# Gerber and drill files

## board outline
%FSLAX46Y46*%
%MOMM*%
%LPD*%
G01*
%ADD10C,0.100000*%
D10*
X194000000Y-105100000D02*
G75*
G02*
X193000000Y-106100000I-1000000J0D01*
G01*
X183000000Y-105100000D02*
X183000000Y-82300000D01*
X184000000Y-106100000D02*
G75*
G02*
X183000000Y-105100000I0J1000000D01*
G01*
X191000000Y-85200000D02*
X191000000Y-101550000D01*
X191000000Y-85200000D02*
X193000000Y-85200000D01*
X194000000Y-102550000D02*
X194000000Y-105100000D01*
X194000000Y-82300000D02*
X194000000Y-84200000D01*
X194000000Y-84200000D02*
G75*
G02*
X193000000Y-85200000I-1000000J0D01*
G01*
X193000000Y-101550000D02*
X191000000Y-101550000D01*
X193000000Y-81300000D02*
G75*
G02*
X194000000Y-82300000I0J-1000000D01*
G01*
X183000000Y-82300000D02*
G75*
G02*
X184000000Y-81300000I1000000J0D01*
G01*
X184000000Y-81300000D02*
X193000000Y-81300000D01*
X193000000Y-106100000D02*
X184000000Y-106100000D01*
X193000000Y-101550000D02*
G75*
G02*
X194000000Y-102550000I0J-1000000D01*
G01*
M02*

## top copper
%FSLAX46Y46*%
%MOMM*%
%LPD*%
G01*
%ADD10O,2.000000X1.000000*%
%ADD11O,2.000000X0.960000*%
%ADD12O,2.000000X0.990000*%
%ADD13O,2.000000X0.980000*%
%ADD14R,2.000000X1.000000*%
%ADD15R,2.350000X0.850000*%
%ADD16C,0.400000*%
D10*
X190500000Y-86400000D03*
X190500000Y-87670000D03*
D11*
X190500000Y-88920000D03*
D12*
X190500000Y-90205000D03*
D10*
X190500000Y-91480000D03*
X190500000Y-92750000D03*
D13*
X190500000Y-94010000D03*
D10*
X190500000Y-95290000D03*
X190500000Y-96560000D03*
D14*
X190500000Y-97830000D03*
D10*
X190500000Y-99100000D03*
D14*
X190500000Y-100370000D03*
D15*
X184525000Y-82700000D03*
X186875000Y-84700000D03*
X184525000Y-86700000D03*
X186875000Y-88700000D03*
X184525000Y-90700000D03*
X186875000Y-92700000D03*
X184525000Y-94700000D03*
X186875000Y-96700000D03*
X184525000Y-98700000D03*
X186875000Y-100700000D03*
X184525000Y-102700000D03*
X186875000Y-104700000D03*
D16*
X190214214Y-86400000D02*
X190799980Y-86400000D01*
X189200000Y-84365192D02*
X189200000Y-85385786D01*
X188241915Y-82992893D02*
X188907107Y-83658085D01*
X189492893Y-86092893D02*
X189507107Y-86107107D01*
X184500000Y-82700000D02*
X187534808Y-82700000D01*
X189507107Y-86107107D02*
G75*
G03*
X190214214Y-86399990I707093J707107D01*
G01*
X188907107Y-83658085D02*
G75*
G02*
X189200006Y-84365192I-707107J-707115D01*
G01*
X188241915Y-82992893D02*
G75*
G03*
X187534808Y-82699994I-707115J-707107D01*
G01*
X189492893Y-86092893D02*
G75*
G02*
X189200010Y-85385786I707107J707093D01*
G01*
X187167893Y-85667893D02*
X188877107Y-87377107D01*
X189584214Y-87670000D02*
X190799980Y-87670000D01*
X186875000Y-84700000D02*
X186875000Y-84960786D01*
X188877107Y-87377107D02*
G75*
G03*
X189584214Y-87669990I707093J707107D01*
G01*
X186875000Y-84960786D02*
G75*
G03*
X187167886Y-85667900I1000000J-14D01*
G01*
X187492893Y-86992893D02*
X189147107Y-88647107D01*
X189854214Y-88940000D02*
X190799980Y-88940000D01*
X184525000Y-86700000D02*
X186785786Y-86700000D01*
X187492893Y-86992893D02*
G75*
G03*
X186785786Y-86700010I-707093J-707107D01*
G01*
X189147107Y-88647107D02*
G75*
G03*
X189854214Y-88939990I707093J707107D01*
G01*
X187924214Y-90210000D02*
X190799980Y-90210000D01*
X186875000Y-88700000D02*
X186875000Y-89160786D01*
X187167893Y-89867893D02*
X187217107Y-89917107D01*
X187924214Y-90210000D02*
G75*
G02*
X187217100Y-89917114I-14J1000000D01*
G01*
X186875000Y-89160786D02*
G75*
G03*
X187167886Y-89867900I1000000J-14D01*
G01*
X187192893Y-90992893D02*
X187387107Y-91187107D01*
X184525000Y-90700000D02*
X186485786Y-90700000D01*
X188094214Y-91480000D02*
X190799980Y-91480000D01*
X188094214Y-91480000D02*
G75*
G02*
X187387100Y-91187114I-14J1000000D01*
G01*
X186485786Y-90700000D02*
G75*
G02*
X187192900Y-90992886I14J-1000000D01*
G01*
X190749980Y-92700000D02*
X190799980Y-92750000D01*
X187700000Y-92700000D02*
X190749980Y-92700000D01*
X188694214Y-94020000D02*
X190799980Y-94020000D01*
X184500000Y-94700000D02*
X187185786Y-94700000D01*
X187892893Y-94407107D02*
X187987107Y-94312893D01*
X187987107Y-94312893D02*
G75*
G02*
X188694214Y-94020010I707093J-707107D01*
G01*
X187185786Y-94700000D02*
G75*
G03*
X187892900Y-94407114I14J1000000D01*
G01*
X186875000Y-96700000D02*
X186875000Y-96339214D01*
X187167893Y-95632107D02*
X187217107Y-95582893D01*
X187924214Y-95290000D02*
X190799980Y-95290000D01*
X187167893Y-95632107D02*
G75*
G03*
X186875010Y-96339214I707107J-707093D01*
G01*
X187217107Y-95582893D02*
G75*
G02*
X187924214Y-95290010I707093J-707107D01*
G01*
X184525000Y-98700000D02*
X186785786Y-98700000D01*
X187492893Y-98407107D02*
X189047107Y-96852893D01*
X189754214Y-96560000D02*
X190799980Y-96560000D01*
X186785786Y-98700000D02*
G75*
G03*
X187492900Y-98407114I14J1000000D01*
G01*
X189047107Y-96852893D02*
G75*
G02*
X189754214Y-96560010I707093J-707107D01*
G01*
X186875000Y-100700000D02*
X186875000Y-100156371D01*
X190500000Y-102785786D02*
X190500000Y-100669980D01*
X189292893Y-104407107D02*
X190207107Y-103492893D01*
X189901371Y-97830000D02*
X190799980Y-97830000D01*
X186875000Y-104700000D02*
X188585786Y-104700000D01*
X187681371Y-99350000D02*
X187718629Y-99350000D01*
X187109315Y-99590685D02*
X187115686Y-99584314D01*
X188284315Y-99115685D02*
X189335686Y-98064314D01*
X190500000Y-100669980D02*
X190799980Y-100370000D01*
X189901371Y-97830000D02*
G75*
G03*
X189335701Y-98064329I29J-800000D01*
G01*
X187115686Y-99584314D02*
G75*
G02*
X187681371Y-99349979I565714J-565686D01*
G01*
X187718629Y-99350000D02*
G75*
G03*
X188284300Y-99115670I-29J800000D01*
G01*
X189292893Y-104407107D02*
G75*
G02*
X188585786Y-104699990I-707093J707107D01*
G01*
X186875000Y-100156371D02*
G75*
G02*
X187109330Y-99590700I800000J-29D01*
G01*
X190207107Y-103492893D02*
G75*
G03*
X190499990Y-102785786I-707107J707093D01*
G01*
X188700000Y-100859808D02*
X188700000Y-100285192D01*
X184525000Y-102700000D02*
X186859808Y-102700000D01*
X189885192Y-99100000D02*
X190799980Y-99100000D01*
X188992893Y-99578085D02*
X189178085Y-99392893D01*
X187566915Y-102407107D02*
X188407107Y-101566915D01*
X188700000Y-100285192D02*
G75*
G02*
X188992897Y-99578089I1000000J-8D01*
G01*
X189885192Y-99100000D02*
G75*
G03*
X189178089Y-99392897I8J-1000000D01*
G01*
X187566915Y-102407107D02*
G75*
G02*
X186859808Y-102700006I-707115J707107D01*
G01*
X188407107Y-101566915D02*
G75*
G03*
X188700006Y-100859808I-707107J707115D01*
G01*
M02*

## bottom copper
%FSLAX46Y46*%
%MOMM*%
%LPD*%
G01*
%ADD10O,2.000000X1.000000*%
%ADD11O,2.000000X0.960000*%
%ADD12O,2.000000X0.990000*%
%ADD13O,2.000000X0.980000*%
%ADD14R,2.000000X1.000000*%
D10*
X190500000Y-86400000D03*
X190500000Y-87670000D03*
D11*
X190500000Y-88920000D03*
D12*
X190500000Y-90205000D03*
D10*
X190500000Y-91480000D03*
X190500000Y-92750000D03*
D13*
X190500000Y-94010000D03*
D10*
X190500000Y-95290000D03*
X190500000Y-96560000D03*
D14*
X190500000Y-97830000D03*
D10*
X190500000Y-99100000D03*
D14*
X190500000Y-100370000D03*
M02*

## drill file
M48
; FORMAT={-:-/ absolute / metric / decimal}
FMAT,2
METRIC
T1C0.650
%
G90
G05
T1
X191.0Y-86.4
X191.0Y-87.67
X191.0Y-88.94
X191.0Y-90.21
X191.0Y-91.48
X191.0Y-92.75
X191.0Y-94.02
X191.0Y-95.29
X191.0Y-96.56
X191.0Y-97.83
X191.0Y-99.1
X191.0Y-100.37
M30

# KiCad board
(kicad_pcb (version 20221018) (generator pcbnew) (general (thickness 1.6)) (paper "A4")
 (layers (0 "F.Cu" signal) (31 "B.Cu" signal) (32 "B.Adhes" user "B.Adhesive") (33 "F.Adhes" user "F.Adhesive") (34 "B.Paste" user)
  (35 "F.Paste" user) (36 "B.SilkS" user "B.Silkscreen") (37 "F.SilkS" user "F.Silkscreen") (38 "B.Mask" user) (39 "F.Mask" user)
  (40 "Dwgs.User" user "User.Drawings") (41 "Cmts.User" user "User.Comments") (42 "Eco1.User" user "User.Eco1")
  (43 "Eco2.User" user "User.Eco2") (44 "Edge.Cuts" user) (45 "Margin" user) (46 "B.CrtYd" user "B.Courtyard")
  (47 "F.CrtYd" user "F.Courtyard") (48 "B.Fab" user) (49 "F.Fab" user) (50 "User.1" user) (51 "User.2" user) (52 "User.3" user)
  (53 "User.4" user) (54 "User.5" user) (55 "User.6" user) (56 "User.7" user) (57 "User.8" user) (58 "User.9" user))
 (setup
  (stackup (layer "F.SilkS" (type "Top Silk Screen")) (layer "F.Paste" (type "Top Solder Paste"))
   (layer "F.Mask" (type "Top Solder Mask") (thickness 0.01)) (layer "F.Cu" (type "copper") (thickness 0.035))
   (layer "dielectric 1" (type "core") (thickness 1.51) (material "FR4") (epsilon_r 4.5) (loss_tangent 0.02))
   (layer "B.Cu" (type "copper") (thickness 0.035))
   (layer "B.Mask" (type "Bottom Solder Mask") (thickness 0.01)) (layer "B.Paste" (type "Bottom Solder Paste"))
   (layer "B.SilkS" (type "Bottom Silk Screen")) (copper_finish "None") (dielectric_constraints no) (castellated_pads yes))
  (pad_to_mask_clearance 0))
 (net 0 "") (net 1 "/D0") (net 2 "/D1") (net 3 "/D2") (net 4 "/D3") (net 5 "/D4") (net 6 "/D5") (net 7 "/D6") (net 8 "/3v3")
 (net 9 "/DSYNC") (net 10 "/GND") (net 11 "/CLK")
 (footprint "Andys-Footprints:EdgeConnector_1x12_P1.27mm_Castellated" (layer "F.Cu") (at 191 86.4)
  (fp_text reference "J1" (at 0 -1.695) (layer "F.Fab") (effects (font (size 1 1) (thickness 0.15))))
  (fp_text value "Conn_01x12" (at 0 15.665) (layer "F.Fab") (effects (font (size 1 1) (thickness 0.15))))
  (pad "1" thru_hole oval (at 0 0) (size 2 1) (drill 0.65 (offset -0.5 0)) (layers "*.Cu" "*.Mask") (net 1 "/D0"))
  (pad "2" thru_hole oval (at 0 1.27) (size 2 1) (drill 0.65 (offset -0.5 0)) (layers "*.Cu" "*.Mask") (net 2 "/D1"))
  (pad "3" thru_hole oval (at 0 2.54) (size 2 0.96) (drill 0.65 (offset -0.5 -0.02)) (layers "*.Cu" "*.Mask") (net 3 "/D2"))
  (pad "4" thru_hole oval (at 0 3.81) (size 2 0.99) (drill 0.65 (offset -0.5 -0.005)) (layers "*.Cu" "*.Mask") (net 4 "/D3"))
  (pad "5" thru_hole oval (at 0 5.08) (size 2 1) (drill 0.65 (offset -0.5 0)) (layers "*.Cu" "*.Mask") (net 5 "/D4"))
  (pad "6" thru_hole oval (at 0 6.35) (size 2 1) (drill 0.65 (offset -0.5 0)) (layers "*.Cu" "*.Mask") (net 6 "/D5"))
  (pad "7" thru_hole oval (at 0 7.62) (size 2 0.98) (drill 0.65 (offset -0.5 -0.01)) (layers "*.Cu" "*.Mask") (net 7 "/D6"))
  (pad "8" thru_hole oval (at 0 8.89) (size 2 1) (drill 0.65 (offset -0.5 0)) (layers "*.Cu" "*.Mask") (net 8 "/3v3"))
  (pad "9" thru_hole oval (at 0 10.16) (size 2 1) (drill 0.65 (offset -0.5 0)) (layers "*.Cu" "*.Mask") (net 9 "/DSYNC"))
  (pad "10" thru_hole rect (at 0 11.43) (size 2 1) (drill 0.65 (offset -0.5 0)) (layers "*.Cu" "*.Mask") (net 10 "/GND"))
  (pad "11" thru_hole oval (at 0 12.7) (size 2 1) (drill 0.65 (offset -0.5 0)) (layers "*.Cu" "*.Mask") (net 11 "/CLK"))
  (pad "12" thru_hole rect (at 0 13.97) (size 2 1) (drill 0.65 (offset -0.5 0)) (layers "*.Cu" "*.Mask") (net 10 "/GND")))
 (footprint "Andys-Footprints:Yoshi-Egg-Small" (layer "F.Cu") (at 191.7 103.8)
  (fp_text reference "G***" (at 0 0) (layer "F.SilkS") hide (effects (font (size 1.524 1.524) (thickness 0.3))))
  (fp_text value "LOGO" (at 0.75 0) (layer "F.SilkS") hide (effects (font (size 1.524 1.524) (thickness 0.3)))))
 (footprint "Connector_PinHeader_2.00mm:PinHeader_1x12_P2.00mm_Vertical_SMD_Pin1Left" (layer "F.Cu") (at 185.7 93.7)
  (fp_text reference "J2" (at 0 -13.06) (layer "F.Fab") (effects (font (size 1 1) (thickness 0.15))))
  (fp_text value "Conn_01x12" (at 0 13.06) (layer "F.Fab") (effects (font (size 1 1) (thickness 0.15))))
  (pad "1" smd rect (at -1.175 -11) (size 2.35 0.85) (layers "F.Cu" "F.Paste" "F.Mask") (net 1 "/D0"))
  (pad "2" smd rect (at 1.175 -9) (size 2.35 0.85) (layers "F.Cu" "F.Paste" "F.Mask") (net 2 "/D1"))
  (pad "3" smd rect (at -1.175 -7) (size 2.35 0.85) (layers "F.Cu" "F.Paste" "F.Mask") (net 3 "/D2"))
  (pad "4" smd rect (at 1.175 -5) (size 2.35 0.85) (layers "F.Cu" "F.Paste" "F.Mask") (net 4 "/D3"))
  (pad "5" smd rect (at -1.175 -3) (size 2.35 0.85) (layers "F.Cu" "F.Paste" "F.Mask") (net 5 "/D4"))
  (pad "6" smd rect (at 1.175 -1) (size 2.35 0.85) (layers "F.Cu" "F.Paste" "F.Mask") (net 6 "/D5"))
  (pad "7" smd rect (at -1.175 1) (size 2.35 0.85) (layers "F.Cu" "F.Paste" "F.Mask") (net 7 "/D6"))
  (pad "8" smd rect (at 1.175 3) (size 2.35 0.85) (layers "F.Cu" "F.Paste" "F.Mask") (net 8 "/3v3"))
  (pad "9" smd rect (at -1.175 5) (size 2.35 0.85) (layers "F.Cu" "F.Paste" "F.Mask") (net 9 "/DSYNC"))
  (pad "10" smd rect (at 1.175 7) (size 2.35 0.85) (layers "F.Cu" "F.Paste" "F.Mask") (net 10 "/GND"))
  (pad "11" smd rect (at -1.175 9) (size 2.35 0.85) (layers "F.Cu" "F.Paste" "F.Mask") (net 11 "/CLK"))
  (pad "12" smd rect (at 1.175 11) (size 2.35 0.85) (layers "F.Cu" "F.Paste" "F.Mask") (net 10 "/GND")))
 (gr_arc (start 194 105.1) (mid 193.707107 105.807107) (end 193 106.1) (stroke (width 0.1) (type solid)) (layer "Edge.Cuts"))
 (gr_line (start 183 105.1) (end 183 82.3) (stroke (width 0.1) (type solid)) (layer "Edge.Cuts"))
 (gr_arc (start 184 106.1) (mid 183.292893 105.807107) (end 183 105.1) (stroke (width 0.1) (type solid)) (layer "Edge.Cuts"))
 (gr_line (start 191 85.2) (end 191 101.55) (stroke (width 0.1) (type solid)) (layer "Edge.Cuts"))
 (gr_line (start 191 85.2) (end 193 85.2) (stroke (width 0.1) (type solid)) (layer "Edge.Cuts"))
 (gr_line (start 194 102.55) (end 194 105.1) (stroke (width 0.1) (type solid)) (layer "Edge.Cuts"))
 (gr_line (start 194 82.3) (end 194 84.2) (stroke (width 0.1) (type solid)) (layer "Edge.Cuts"))
 (gr_arc (start 194 84.2) (mid 193.707107 84.907107) (end 193 85.2) (stroke (width 0.1) (type solid)) (layer "Edge.Cuts"))
 (gr_line (start 193 101.55) (end 191 101.55) (stroke (width 0.1) (type solid)) (layer "Edge.Cuts"))
 (gr_arc (start 193 81.3) (mid 193.707107 81.592893) (end 194 82.3) (stroke (width 0.1) (type solid)) (layer "Edge.Cuts"))
 (gr_arc (start 183 82.3) (mid 183.292893 81.592893) (end 184 81.3) (stroke (width 0.1) (type solid)) (layer "Edge.Cuts"))
 (gr_line (start 184 81.3) (end 193 81.3) (stroke (width 0.1) (type solid)) (layer "Edge.Cuts"))
 (gr_line (start 193 106.1) (end 184 106.1) (stroke (width 0.1) (type solid)) (layer "Edge.Cuts"))
 (gr_arc (start 193 101.55) (mid 193.707107 101.842893) (end 194 102.55) (stroke (width 0.1) (type solid)) (layer "Edge.Cuts"))
 (segment (start 190.214214 86.4) (end 190.79998 86.4) (width 0.4) (layer "F.Cu") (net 1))
 (segment (start 189.2 84.365192) (end 189.2 85.385786) (width 0.4) (layer "F.Cu") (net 1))
 (segment (start 188.241915 82.992893) (end 188.907107 83.658085) (width 0.4) (layer "F.Cu") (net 1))
 (segment (start 189.492893 86.092893) (end 189.507107 86.107107) (width 0.4) (layer "F.Cu") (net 1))
 (segment (start 184.5 82.7) (end 187.534808 82.7) (width 0.4) (layer "F.Cu") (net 1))
 (arc (start 189.507107 86.107107) (mid 189.83153 86.32388) (end 190.214214 86.4) (width 0.4) (layer "F.Cu") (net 1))
 (arc (start 188.907107 83.658085) (mid 189.12388 83.982508) (end 189.2 84.365192) (width 0.4) (layer "F.Cu") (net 1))
 (arc (start 188.241915 82.992893) (mid 187.917492 82.77612) (end 187.534808 82.7) (width 0.4) (layer "F.Cu") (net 1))
 (arc (start 189.492893 86.092893) (mid 189.27612 85.76847) (end 189.2 85.385786) (width 0.4) (layer "F.Cu") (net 1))
 (segment (start 187.167893 85.667893) (end 188.877107 87.377107) (width 0.4) (layer "F.Cu") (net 2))
 (segment (start 189.584214 87.67) (end 190.79998 87.67) (width 0.4) (layer "F.Cu") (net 2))
 (segment (start 186.875 84.7) (end 186.875 84.960786) (width 0.4) (layer "F.Cu") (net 2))
 (arc (start 188.877107 87.377107) (mid 189.20153 87.59388) (end 189.584214 87.67) (width 0.4) (layer "F.Cu") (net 2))
 (arc (start 186.875 84.960786) (mid 186.95112 85.343469) (end 187.167893 85.667893) (width 0.4) (layer "F.Cu") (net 2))
 (segment (start 187.492893 86.992893) (end 189.147107 88.647107) (width 0.4) (layer "F.Cu") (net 3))
 (segment (start 189.854214 88.94) (end 190.79998 88.94) (width 0.4) (layer "F.Cu") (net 3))
 (segment (start 184.525 86.7) (end 186.785786 86.7) (width 0.4) (layer "F.Cu") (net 3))
 (arc (start 187.492893 86.992893) (mid 187.16847 86.77612) (end 186.785786 86.7) (width 0.4) (layer "F.Cu") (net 3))
 (arc (start 189.147107 88.647107) (mid 189.47153 88.86388) (end 189.854214 88.94) (width 0.4) (layer "F.Cu") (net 3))
 (segment (start 187.924214 90.21) (end 190.79998 90.21) (width 0.4) (layer "F.Cu") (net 4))
 (segment (start 186.875 88.7) (end 186.875 89.160786) (width 0.4) (layer "F.Cu") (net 4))
 (segment (start 187.167893 89.867893) (end 187.217107 89.917107) (width 0.4) (layer "F.Cu") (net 4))
 (arc (start 187.924214 90.21) (mid 187.541531 90.13388) (end 187.217107 89.917107) (width 0.4) (layer "F.Cu") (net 4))
 (arc (start 186.875 89.160786) (mid 186.95112 89.543469) (end 187.167893 89.867893) (width 0.4) (layer "F.Cu") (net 4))
 (segment (start 187.192893 90.992893) (end 187.387107 91.187107) (width 0.4) (layer "F.Cu") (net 5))
 (segment (start 184.525 90.7) (end 186.485786 90.7) (width 0.4) (layer "F.Cu") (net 5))
 (segment (start 188.094214 91.48) (end 190.79998 91.48) (width 0.4) (layer "F.Cu") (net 5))
 (arc (start 188.094214 91.48) (mid 187.711531 91.40388) (end 187.387107 91.187107) (width 0.4) (layer "F.Cu") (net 5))
 (arc (start 186.485786 90.7) (mid 186.868469 90.77612) (end 187.192893 90.992893) (width 0.4) (layer "F.Cu") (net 5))
 (segment (start 190.74998 92.7) (end 190.79998 92.75) (width 0.4) (layer "F.Cu") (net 6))
 (segment (start 187.7 92.7) (end 190.74998 92.7) (width 0.4) (layer "F.Cu") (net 6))
 (segment (start 188.694214 94.02) (end 190.79998 94.02) (width 0.4) (layer "F.Cu") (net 7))
 (segment (start 184.5 94.7) (end 187.185786 94.7) (width 0.4) (layer "F.Cu") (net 7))
 (segment (start 187.892893 94.407107) (end 187.987107 94.312893) (width 0.4) (layer "F.Cu") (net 7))
 (arc (start 187.987107 94.312893) (mid 188.31153 94.09612) (end 188.694214 94.02) (width 0.4) (layer "F.Cu") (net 7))
 (arc (start 187.185786 94.7) (mid 187.568469 94.62388) (end 187.892893 94.407107) (width 0.4) (layer "F.Cu") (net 7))
 (segment (start 186.875 96.7) (end 186.875 96.339214) (width 0.4) (layer "F.Cu") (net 8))
 (segment (start 187.167893 95.632107) (end 187.217107 95.582893) (width 0.4) (layer "F.Cu") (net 8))
 (segment (start 187.924214 95.29) (end 190.79998 95.29) (width 0.4) (layer "F.Cu") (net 8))
 (arc (start 187.167893 95.632107) (mid 186.95112 95.95653) (end 186.875 96.339214) (width 0.4) (layer "F.Cu") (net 8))
 (arc (start 187.217107 95.582893) (mid 187.54153 95.36612) (end 187.924214 95.29) (width 0.4) (layer "F.Cu") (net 8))
 (segment (start 184.525 98.7) (end 186.785786 98.7) (width 0.4) (layer "F.Cu") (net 9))
 (segment (start 187.492893 98.407107) (end 189.047107 96.852893) (width 0.4) (layer "F.Cu") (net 9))
 (segment (start 189.754214 96.56) (end 190.79998 96.56) (width 0.4) (layer "F.Cu") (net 9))
 (arc (start 186.785786 98.7) (mid 187.168469 98.62388) (end 187.492893 98.407107) (width 0.4) (layer "F.Cu") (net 9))
 (arc (start 189.047107 96.852893) (mid 189.37153 96.63612) (end 189.754214 96.56) (width 0.4) (layer "F.Cu") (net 9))
 (segment (start 186.875 100.7) (end 186.875 100.156371) (width 0.4) (layer "F.Cu") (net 10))
 (segment (start 190.5 102.785786) (end 190.5 100.66998) (width 0.4) (layer "F.Cu") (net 10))
 (segment (start 189.292893 104.407107) (end 190.207107 103.492893) (width 0.4) (layer "F.Cu") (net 10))
 (segment (start 189.901371 97.83) (end 190.79998 97.83) (width 0.4) (layer "F.Cu") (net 10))
 (segment (start 186.875 104.7) (end 188.585786 104.7) (width 0.4) (layer "F.Cu") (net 10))
 (segment (start 187.681371 99.35) (end 187.718629 99.35) (width 0.4) (layer "F.Cu") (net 10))
 (segment (start 187.109315 99.590685) (end 187.115686 99.584314) (width 0.4) (layer "F.Cu") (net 10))
 (segment (start 188.284315 99.115685) (end 189.335686 98.064314) (width 0.4) (layer "F.Cu") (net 10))
 (segment (start 190.5 100.66998) (end 190.79998 100.37) (width 0.4) (layer "F.Cu") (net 10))
 (arc (start 189.901371 97.83) (mid 189.595225 97.890896) (end 189.335686 98.064314) (width 0.4) (layer "F.Cu") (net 10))
 (arc (start 187.115686 99.584314) (mid 187.375225 99.410896) (end 187.681371 99.35) (width 0.4) (layer "F.Cu") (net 10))
 (arc (start 187.718629 99.35) (mid 188.024776 99.289103) (end 188.284315 99.115685) (width 0.4) (layer "F.Cu") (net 10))
 (arc (start 189.292893 104.407107) (mid 188.96847 104.62388) (end 188.585786 104.7) (width 0.4) (layer "F.Cu") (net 10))
 (arc (start 186.875 100.156371) (mid 186.935897 99.850224) (end 187.109315 99.590685) (width 0.4) (layer "F.Cu") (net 10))
 (arc (start 190.207107 103.492893) (mid 190.42388 103.16847) (end 190.5 102.785786) (width 0.4) (layer "F.Cu") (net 10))
 (segment (start 188.7 100.859808) (end 188.7 100.285192) (width 0.4) (layer "F.Cu") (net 11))
 (segment (start 184.525 102.7) (end 186.859808 102.7) (width 0.4) (layer "F.Cu") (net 11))
 (segment (start 189.885192 99.1) (end 190.79998 99.1) (width 0.4) (layer "F.Cu") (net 11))
 (segment (start 188.992893 99.578085) (end 189.178085 99.392893) (width 0.4) (layer "F.Cu") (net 11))
 (segment (start 187.566915 102.407107) (end 188.407107 101.566915) (width 0.4) (layer "F.Cu") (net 11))
 (arc (start 188.7 100.285192) (mid 188.77612 99.902509) (end 188.992893 99.578085) (width 0.4) (layer "F.Cu") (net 11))
 (arc (start 189.885192 99.1) (mid 189.502509 99.17612) (end 189.178085 99.392893) (width 0.4) (layer "F.Cu") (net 11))
 (arc (start 187.566915 102.407107) (mid 187.242492 102.62388) (end 186.859808 102.7) (width 0.4) (layer "F.Cu") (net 11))
 (arc (start 188.407107 101.566915) (mid 188.62388 101.242492) (end 188.7 100.859808) (width 0.4) (layer "F.Cu") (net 11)))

